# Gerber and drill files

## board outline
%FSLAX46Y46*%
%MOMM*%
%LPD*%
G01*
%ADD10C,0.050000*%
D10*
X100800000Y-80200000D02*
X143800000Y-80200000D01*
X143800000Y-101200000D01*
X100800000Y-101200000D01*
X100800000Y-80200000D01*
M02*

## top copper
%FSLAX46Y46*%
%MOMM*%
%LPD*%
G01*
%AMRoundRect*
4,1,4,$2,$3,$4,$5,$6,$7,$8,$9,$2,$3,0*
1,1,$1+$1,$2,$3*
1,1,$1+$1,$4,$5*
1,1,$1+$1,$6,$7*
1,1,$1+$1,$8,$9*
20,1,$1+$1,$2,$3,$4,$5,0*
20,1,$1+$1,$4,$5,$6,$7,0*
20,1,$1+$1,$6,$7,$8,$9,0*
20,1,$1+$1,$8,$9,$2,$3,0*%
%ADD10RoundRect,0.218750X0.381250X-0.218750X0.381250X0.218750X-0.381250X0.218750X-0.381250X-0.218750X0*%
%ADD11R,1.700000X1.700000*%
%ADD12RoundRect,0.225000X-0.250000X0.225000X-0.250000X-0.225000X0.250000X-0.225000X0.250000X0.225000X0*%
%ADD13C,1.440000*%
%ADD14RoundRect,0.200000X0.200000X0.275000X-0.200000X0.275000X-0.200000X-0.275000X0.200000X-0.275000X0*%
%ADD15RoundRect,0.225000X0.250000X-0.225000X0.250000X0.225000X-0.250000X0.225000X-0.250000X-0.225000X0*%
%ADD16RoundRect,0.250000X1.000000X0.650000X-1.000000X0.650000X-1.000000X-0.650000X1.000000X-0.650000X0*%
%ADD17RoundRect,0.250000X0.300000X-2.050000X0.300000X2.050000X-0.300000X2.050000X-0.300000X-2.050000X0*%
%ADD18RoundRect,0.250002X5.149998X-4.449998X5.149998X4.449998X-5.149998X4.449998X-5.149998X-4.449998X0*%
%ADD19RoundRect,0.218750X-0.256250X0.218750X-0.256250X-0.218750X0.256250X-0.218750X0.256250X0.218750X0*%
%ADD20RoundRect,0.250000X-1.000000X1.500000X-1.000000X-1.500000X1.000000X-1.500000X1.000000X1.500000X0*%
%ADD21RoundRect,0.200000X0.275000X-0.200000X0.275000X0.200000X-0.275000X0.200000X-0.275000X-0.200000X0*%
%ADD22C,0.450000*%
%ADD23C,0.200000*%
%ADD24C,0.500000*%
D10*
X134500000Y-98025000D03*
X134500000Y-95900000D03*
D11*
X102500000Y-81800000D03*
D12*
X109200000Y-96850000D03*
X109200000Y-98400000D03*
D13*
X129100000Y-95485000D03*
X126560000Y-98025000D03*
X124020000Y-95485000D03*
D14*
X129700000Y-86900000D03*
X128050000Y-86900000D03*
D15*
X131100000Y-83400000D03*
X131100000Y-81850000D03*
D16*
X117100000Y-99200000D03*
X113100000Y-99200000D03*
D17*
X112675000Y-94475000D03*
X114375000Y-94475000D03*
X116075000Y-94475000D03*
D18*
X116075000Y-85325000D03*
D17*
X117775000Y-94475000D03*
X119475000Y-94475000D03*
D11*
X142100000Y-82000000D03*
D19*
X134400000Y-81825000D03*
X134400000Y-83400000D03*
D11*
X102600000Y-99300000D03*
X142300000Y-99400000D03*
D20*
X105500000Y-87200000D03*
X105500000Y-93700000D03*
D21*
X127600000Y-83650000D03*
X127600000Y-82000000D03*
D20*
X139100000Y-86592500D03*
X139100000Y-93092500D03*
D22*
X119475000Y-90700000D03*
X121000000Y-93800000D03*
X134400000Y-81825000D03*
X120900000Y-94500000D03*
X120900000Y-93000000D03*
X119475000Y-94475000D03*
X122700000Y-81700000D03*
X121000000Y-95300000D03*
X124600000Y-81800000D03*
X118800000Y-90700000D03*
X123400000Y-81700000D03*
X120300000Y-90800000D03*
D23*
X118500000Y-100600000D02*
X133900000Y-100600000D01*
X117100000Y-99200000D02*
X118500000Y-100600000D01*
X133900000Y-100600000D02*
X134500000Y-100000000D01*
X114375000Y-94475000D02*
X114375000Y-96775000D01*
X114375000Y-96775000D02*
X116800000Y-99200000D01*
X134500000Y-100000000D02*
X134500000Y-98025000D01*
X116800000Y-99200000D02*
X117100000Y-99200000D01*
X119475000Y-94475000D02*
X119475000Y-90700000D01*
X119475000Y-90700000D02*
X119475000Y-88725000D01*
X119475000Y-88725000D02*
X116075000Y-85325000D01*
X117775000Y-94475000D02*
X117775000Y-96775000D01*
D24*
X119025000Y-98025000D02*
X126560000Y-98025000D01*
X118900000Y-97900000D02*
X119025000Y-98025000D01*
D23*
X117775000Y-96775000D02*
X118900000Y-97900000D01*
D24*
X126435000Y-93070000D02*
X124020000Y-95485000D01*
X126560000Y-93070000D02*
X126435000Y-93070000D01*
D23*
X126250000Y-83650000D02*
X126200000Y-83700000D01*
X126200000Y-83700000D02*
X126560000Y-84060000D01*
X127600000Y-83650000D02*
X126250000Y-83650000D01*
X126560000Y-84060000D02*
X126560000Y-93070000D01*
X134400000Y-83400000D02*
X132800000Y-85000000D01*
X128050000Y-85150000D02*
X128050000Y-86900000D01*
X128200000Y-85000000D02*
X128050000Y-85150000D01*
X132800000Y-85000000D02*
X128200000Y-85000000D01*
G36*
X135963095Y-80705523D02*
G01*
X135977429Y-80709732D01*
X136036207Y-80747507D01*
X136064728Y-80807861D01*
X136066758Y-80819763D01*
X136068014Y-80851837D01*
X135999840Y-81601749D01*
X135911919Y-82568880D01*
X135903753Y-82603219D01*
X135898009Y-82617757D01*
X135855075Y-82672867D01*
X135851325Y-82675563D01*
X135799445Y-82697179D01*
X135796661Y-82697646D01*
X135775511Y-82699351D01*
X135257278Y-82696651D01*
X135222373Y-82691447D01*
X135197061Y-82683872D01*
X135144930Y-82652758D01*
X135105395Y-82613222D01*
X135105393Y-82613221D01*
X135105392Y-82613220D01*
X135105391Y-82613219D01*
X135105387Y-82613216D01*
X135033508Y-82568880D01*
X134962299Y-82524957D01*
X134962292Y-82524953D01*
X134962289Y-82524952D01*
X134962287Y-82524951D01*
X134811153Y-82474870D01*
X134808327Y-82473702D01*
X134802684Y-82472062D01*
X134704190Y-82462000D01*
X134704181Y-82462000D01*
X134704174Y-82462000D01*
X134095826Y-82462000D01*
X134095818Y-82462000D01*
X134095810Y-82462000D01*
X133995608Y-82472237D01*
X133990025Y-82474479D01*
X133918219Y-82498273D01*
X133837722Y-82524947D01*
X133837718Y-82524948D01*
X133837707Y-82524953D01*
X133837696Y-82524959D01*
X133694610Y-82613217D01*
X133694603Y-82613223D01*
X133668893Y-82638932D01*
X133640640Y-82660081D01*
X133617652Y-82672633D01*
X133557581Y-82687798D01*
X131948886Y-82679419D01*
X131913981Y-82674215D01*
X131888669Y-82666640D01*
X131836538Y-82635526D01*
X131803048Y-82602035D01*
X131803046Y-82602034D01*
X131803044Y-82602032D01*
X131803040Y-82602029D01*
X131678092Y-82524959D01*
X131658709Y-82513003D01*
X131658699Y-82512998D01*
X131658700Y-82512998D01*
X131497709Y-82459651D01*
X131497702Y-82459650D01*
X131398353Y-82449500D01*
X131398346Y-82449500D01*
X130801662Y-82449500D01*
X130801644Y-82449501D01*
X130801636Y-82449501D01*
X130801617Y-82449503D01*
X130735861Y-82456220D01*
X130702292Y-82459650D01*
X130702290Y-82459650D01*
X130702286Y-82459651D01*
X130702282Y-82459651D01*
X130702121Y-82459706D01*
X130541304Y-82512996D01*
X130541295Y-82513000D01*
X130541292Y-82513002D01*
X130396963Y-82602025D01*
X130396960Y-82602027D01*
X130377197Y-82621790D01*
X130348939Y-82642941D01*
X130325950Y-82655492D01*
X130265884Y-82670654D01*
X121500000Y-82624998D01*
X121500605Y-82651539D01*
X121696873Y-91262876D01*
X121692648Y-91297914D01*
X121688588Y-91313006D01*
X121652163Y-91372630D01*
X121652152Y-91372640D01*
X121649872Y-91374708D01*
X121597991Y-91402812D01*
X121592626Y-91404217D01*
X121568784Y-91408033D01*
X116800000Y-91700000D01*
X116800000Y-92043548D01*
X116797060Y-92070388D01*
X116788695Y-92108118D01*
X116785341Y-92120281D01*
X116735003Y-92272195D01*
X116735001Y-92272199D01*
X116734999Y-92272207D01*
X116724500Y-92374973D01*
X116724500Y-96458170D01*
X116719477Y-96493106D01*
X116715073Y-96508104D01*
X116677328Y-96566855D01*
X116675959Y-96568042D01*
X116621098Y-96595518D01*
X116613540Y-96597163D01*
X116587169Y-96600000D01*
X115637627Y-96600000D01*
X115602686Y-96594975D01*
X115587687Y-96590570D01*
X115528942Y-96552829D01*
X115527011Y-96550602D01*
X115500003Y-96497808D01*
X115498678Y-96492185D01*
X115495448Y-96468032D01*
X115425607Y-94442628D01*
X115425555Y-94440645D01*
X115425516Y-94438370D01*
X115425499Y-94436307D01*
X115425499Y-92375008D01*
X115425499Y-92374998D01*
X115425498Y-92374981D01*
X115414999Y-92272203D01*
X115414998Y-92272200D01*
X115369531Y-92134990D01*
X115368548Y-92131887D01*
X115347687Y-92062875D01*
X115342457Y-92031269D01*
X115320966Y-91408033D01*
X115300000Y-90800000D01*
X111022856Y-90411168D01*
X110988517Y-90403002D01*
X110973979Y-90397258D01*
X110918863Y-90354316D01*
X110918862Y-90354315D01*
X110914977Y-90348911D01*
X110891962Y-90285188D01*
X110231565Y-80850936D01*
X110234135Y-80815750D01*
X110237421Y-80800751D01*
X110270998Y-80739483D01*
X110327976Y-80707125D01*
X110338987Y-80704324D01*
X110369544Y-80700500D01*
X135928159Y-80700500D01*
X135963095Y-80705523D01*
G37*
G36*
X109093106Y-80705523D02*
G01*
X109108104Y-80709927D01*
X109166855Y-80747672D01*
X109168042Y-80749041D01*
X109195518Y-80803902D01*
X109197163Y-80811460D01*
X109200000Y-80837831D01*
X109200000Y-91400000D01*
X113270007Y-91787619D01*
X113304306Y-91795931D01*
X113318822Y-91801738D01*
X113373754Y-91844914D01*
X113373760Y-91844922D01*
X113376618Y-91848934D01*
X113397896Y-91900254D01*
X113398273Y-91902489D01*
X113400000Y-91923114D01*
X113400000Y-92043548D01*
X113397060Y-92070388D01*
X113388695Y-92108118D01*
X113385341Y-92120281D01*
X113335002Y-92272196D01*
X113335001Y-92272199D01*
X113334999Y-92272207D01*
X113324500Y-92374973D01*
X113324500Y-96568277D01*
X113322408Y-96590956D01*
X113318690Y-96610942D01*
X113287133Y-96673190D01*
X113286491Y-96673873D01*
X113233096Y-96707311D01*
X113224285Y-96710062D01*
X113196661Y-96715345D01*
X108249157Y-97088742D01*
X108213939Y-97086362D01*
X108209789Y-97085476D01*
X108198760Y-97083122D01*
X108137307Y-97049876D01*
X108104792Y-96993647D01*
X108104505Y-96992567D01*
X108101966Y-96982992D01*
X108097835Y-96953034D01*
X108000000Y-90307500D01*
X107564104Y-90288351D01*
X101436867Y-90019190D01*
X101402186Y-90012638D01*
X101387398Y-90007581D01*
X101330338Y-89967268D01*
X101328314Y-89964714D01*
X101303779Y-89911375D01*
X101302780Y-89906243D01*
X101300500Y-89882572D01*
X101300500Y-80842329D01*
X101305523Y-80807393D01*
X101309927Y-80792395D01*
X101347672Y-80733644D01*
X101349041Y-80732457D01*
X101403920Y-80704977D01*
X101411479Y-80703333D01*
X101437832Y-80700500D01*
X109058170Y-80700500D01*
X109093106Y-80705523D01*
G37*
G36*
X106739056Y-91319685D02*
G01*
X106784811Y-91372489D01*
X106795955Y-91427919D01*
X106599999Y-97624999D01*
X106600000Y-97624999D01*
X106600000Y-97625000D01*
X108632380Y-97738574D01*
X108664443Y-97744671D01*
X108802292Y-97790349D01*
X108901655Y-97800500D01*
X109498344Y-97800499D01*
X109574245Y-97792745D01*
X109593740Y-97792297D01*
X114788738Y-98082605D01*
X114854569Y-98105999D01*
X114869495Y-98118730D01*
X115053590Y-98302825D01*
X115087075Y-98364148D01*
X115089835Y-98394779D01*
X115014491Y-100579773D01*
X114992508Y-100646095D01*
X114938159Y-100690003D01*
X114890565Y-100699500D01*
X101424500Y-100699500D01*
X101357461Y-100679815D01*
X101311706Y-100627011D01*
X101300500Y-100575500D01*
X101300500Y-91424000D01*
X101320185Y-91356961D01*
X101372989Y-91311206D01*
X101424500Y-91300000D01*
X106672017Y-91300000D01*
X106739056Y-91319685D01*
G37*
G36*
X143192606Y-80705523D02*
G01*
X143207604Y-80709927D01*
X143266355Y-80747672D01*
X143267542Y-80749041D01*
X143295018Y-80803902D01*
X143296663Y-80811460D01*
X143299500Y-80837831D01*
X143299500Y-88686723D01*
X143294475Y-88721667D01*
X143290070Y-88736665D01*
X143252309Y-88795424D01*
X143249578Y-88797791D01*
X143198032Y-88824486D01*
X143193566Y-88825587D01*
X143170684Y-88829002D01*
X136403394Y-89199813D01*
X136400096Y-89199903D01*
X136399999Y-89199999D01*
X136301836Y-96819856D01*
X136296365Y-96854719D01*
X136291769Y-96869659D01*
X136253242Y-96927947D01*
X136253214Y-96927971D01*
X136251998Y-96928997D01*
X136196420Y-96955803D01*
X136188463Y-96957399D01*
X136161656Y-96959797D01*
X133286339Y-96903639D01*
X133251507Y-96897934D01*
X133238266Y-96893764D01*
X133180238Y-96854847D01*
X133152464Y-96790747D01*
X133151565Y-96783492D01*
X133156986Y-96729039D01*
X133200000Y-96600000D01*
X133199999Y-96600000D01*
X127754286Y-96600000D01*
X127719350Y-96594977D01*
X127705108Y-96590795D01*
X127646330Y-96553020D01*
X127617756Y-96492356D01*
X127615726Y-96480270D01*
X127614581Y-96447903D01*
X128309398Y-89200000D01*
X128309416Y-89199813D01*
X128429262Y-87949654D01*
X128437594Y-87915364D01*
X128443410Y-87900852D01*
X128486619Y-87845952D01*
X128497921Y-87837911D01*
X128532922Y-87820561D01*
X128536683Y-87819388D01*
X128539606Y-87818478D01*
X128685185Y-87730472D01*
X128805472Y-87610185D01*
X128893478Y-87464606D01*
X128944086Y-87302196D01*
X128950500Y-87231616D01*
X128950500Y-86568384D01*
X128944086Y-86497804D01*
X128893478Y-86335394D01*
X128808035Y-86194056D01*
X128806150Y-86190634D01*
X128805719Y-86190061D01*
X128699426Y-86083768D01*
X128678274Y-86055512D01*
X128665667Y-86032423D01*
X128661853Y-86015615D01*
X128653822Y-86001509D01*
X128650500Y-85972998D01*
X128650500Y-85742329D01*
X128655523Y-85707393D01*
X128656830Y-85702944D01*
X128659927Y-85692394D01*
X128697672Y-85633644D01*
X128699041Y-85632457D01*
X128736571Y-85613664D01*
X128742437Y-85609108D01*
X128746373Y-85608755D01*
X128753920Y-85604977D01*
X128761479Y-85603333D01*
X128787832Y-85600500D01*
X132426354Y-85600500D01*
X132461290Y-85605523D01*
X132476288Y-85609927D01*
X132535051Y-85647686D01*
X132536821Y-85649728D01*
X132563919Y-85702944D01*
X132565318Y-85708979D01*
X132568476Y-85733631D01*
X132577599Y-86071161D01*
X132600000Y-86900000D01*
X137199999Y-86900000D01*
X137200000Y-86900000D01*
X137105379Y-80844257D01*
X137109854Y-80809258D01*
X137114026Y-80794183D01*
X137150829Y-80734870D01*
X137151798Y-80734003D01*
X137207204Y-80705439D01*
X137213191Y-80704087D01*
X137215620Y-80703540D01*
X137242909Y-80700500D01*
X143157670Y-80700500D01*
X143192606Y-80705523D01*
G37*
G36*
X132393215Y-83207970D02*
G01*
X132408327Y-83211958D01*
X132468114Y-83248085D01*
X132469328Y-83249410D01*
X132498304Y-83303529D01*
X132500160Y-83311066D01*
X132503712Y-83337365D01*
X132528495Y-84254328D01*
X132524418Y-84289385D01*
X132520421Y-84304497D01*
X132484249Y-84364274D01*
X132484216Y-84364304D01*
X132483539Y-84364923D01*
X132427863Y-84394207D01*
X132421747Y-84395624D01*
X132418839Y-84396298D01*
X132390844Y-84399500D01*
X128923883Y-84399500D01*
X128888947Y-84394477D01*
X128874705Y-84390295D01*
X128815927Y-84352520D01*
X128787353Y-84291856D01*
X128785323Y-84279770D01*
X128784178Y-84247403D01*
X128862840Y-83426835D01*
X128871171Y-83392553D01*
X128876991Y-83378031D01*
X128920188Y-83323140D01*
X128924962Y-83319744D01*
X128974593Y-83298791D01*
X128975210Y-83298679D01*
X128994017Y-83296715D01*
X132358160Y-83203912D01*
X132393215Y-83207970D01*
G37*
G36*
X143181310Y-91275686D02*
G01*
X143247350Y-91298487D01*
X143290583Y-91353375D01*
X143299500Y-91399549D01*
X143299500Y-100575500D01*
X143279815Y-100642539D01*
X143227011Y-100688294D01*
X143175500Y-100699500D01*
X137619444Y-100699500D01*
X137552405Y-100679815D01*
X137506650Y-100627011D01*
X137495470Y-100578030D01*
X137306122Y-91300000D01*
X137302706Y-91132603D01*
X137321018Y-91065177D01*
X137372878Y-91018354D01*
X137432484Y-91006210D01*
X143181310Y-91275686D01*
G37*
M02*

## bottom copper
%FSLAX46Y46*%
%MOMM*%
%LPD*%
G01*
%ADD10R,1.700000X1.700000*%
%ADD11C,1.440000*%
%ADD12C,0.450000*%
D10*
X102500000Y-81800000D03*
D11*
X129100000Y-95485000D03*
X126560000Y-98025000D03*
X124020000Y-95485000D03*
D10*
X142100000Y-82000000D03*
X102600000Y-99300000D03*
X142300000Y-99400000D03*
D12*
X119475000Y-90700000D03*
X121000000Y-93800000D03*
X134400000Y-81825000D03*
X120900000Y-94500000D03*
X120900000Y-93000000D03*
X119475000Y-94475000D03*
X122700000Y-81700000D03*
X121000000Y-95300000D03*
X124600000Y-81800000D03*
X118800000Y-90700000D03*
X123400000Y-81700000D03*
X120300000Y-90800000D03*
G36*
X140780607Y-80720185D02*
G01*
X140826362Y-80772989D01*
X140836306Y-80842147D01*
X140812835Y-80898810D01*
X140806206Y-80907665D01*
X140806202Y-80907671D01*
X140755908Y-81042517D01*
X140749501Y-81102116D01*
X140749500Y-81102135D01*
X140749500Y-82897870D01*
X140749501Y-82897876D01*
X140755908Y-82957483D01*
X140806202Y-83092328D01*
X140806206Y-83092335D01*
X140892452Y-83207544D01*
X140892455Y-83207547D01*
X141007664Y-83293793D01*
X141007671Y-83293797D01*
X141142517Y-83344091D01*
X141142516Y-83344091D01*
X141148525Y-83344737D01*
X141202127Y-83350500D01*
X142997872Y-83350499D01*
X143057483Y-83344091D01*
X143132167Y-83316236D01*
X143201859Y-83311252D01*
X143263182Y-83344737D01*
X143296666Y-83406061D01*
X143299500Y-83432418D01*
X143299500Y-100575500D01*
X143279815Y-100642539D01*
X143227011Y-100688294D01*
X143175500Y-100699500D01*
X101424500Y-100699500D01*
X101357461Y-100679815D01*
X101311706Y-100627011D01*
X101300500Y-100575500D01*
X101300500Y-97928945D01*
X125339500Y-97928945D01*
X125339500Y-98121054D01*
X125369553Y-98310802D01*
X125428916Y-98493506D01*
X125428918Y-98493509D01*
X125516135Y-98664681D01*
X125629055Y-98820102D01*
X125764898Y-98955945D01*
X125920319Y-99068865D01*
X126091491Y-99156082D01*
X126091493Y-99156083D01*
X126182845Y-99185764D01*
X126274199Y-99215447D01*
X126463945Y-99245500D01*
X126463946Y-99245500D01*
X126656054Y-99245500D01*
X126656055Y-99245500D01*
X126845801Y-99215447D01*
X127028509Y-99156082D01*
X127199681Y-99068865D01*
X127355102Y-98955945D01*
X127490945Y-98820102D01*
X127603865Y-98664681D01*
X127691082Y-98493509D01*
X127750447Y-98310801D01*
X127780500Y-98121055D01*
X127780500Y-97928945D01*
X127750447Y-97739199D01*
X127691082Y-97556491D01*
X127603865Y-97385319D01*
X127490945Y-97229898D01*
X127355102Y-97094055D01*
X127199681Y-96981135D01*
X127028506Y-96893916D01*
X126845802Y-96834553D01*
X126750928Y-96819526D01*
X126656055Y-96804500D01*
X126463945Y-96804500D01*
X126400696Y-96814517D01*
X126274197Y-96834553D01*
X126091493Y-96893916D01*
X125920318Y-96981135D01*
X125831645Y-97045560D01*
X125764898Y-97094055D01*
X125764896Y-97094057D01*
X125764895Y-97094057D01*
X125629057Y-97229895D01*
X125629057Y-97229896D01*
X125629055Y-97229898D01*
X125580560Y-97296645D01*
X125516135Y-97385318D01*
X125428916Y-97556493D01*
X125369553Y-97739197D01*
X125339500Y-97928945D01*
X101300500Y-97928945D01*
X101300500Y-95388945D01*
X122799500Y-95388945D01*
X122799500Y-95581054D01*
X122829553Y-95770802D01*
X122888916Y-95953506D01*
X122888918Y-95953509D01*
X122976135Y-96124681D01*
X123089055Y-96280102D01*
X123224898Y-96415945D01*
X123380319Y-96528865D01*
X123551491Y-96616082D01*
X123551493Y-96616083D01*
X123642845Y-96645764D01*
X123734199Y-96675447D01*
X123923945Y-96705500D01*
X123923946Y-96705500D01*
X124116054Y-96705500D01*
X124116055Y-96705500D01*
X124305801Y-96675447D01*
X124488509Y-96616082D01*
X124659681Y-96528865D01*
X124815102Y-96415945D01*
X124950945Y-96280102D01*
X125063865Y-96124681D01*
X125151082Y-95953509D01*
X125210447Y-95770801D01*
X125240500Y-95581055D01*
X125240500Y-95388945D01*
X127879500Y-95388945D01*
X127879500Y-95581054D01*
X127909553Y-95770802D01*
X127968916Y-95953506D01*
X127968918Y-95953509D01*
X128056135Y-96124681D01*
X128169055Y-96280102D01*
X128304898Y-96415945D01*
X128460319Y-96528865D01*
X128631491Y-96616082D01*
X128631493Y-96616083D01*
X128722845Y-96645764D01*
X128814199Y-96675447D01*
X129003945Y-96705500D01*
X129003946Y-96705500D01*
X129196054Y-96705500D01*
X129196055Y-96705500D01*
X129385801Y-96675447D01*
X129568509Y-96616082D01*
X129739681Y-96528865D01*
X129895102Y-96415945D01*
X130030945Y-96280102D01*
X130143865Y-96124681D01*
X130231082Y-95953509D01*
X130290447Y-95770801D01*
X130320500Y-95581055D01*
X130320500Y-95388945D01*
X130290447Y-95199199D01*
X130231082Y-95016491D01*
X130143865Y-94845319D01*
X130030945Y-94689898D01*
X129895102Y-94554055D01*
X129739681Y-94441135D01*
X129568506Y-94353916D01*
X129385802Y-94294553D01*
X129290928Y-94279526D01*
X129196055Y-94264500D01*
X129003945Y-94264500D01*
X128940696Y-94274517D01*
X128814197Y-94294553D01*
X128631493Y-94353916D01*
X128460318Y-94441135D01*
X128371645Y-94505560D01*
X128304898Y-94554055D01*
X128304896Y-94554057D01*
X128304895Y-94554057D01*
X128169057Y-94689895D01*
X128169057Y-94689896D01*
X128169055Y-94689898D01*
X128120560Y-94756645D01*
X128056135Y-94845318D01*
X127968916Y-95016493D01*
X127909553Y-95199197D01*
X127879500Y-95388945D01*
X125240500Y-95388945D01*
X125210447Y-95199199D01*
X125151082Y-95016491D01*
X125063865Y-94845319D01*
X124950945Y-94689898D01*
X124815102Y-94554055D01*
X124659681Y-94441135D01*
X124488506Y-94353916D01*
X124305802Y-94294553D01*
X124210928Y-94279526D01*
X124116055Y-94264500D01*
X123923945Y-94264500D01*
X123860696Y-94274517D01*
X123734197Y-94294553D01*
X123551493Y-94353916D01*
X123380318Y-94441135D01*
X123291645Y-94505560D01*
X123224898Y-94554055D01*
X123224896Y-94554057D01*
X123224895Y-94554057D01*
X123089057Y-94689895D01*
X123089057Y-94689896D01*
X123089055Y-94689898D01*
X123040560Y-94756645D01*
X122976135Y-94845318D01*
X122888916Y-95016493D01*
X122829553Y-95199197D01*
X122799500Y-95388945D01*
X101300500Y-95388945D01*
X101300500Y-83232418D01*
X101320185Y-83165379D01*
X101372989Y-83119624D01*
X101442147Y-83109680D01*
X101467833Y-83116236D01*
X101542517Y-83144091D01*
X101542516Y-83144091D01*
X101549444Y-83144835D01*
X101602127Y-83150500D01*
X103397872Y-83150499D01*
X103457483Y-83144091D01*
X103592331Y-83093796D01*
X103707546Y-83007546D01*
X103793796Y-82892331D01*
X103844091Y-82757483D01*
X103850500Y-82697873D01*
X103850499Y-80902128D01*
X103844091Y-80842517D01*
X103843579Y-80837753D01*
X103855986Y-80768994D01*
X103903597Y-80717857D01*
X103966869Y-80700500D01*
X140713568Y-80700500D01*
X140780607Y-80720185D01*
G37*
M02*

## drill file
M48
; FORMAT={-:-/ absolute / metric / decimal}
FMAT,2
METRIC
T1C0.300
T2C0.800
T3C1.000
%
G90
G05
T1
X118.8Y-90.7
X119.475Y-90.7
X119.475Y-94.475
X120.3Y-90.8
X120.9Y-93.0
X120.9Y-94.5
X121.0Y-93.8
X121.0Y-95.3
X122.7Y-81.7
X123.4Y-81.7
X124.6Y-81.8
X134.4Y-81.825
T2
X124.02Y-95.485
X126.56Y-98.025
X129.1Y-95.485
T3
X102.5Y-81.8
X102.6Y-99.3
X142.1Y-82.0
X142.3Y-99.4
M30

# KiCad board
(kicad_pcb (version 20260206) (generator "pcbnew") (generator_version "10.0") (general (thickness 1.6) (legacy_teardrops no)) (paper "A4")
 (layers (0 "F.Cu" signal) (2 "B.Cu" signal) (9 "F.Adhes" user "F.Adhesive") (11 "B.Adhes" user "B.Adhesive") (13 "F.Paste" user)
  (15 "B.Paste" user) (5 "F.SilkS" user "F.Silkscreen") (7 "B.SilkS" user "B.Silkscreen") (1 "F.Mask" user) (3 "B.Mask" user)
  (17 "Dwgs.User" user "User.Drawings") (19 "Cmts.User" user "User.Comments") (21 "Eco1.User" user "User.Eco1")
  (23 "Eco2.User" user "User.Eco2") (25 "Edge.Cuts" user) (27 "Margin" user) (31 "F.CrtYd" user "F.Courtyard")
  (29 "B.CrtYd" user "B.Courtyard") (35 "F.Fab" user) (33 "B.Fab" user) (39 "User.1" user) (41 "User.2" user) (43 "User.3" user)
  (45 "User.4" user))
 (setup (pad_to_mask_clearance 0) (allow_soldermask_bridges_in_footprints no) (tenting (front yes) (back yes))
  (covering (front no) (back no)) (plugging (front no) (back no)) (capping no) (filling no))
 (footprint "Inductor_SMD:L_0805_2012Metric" (layer "F.Cu") (at 134.5 96.9625 90)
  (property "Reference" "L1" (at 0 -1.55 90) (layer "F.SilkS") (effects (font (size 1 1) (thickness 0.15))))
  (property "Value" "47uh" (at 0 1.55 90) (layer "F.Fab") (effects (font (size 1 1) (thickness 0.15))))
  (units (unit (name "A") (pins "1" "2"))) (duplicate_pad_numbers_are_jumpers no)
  (pad "1" smd roundrect (at -1.0625 0 90) (size 0.875 1.2) (layers "F.Cu" "F.Mask" "F.Paste") (roundrect_rratio 0.25) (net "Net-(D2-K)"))
  (pad "2" smd roundrect (at 1.0625 0 90) (size 0.875 1.2) (layers "F.Cu" "F.Mask" "F.Paste") (roundrect_rratio 0.25) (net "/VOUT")))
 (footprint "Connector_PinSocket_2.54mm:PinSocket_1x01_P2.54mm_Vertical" (layer "F.Cu") (at 102.5 81.8)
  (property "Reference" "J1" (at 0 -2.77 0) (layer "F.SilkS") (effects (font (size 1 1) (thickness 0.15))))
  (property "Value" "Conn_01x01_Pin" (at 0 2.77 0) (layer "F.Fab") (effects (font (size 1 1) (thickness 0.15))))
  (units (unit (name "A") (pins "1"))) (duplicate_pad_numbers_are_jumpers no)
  (pad "1" thru_hole rect (at 0 0) (size 1.7 1.7) (drill 1) (layers "*.Cu" "*.Mask") (remove_unused_layers no) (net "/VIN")))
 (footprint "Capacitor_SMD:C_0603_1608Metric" (layer "F.Cu") (at 109.2 97.625 -90)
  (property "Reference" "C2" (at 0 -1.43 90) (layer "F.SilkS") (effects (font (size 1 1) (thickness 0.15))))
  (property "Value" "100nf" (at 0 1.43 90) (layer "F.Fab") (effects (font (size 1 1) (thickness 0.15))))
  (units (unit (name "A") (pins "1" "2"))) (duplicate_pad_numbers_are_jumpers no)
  (pad "1" smd roundrect (at -0.775 0 270) (size 0.9 0.95) (layers "F.Cu" "F.Mask" "F.Paste") (roundrect_rratio 0.25) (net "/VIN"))
  (pad "2" smd roundrect (at 0.775 0 270) (size 0.9 0.95) (layers "F.Cu" "F.Mask" "F.Paste") (roundrect_rratio 0.25) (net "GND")))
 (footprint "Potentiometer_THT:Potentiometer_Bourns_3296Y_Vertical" (layer "F.Cu") (at 129.1 95.485)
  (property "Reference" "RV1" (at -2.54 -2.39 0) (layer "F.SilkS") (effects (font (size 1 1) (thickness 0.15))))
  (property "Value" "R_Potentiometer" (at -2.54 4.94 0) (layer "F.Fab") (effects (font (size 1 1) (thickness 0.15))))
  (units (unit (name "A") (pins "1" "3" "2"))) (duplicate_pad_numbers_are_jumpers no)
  (pad "1" thru_hole circle (at 0 0) (size 1.44 1.44) (drill 0.8) (layers "*.Cu" "*.Mask") (remove_unused_layers no) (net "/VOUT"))
  (pad "2" thru_hole circle (at -2.54 2.54) (size 1.44 1.44) (drill 0.8) (layers "*.Cu" "*.Mask") (remove_unused_layers no)
   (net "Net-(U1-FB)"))
  (pad "3" thru_hole circle (at -5.08 0) (size 1.44 1.44) (drill 0.8) (layers "*.Cu" "*.Mask") (remove_unused_layers no)
   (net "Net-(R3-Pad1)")))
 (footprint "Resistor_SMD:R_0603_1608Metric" (layer "F.Cu") (at 128.875 86.9 180)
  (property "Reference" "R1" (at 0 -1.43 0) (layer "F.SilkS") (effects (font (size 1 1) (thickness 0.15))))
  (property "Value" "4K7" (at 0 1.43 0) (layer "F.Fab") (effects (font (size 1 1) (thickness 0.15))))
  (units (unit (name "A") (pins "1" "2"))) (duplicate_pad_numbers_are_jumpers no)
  (pad "1" smd roundrect (at -0.825 0 180) (size 0.8 0.95) (layers "F.Cu" "F.Mask" "F.Paste") (roundrect_rratio 0.25) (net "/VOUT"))
  (pad "2" smd roundrect (at 0.825 0 180) (size 0.8 0.95) (layers "F.Cu" "F.Mask" "F.Paste") (roundrect_rratio 0.25) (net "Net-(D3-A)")))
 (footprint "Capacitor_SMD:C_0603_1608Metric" (layer "F.Cu") (at 131.1 82.625 90)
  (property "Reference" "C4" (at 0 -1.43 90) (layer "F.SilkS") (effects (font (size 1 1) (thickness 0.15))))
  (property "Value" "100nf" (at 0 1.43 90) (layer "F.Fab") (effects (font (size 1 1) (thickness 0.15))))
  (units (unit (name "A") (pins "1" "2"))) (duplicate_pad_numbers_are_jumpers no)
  (pad "1" smd roundrect (at -0.775 0 90) (size 0.9 0.95) (layers "F.Cu" "F.Mask" "F.Paste") (roundrect_rratio 0.25) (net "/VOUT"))
  (pad "2" smd roundrect (at 0.775 0 90) (size 0.9 0.95) (layers "F.Cu" "F.Mask" "F.Paste") (roundrect_rratio 0.25) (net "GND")))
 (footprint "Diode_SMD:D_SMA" (layer "F.Cu") (at 115.1 99.2 180)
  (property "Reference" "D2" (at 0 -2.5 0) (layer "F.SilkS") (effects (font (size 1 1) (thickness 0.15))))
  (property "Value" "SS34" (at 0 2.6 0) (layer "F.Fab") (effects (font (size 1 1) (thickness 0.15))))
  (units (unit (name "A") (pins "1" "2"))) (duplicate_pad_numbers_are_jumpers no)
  (pad "1" smd roundrect (at -2 0 180) (size 2.5 1.8) (layers "F.Cu" "F.Mask" "F.Paste") (roundrect_rratio 0.1388888889) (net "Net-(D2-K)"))
  (pad "2" smd roundrect (at 2 0 180) (size 2.5 1.8) (layers "F.Cu" "F.Mask" "F.Paste") (roundrect_rratio 0.1388888889) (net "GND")))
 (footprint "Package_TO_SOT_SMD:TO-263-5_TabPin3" (layer "F.Cu") (at 116.075 86.825 90)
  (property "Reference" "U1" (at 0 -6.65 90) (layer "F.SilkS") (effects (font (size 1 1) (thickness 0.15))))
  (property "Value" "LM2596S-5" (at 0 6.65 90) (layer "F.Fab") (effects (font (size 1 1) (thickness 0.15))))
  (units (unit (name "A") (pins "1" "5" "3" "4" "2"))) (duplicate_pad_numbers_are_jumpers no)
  (pad "" smd roundrect (at -0.925 -2.775 90) (size 4.55 5.25) (layers "F.Paste") (roundrect_rratio 0.054945))
  (pad "" smd roundrect (at -0.925 2.775 90) (size 4.55 5.25) (layers "F.Paste") (roundrect_rratio 0.054945))
  (pad "" smd roundrect (at 3.925 -2.775 90) (size 4.55 5.25) (layers "F.Paste") (roundrect_rratio 0.054945))
  (pad "" smd roundrect (at 3.925 2.775 90) (size 4.55 5.25) (layers "F.Paste") (roundrect_rratio 0.054945))
  (pad "1" smd roundrect (at -7.65 -3.4 90) (size 4.6 1.1) (layers "F.Cu" "F.Mask" "F.Paste") (roundrect_rratio 0.227273) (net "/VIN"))
  (pad "2" smd roundrect (at -7.65 -1.7 90) (size 4.6 1.1) (layers "F.Cu" "F.Mask" "F.Paste") (roundrect_rratio 0.227273) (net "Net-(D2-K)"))
  (pad "3" smd roundrect (at -7.65 0 90) (size 4.6 1.1) (layers "F.Cu" "F.Mask" "F.Paste") (roundrect_rratio 0.227273) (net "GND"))
  (pad "3" smd roundrect (at 1.5 0 90) (size 9.4 10.8) (layers "F.Cu" "F.Mask") (roundrect_rratio 0.026596) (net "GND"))
  (pad "4" smd roundrect (at -7.65 1.7 90) (size 4.6 1.1) (layers "F.Cu" "F.Mask" "F.Paste") (roundrect_rratio 0.227273) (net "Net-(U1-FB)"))
  (pad "5" smd roundrect (at -7.65 3.4 90) (size 4.6 1.1) (layers "F.Cu" "F.Mask" "F.Paste") (roundrect_rratio 0.227273) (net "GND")))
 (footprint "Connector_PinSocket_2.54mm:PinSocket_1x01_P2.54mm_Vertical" (layer "F.Cu") (at 142.1 82)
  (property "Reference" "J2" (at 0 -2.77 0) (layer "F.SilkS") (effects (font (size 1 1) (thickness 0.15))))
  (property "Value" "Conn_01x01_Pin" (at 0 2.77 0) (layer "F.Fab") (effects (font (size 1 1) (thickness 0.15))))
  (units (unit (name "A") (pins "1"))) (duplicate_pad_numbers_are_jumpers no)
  (pad "1" thru_hole rect (at 0 0) (size 1.7 1.7) (drill 1) (layers "*.Cu" "*.Mask") (remove_unused_layers no) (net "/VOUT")))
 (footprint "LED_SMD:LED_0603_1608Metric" (layer "F.Cu") (at 134.4 82.6125 -90)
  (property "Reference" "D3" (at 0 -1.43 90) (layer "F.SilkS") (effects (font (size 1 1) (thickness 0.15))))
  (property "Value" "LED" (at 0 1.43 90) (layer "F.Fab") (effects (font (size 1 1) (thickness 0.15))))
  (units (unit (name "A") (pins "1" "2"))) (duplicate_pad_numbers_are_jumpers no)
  (pad "1" smd roundrect (at -0.7875 0 270) (size 0.875 0.95) (layers "F.Cu" "F.Mask" "F.Paste") (roundrect_rratio 0.25) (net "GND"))
  (pad "2" smd roundrect (at 0.7875 0 270) (size 0.875 0.95) (layers "F.Cu" "F.Mask" "F.Paste") (roundrect_rratio 0.25) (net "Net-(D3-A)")))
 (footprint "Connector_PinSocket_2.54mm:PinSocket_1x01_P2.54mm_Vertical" (layer "F.Cu") (at 102.6 99.3)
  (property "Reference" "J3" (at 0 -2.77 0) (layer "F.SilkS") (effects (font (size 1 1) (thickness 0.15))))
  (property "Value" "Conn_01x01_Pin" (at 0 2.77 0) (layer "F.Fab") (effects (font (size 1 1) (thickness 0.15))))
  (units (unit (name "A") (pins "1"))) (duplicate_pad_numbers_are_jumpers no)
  (pad "1" thru_hole rect (at 0 0) (size 1.7 1.7) (drill 1) (layers "*.Cu" "*.Mask") (remove_unused_layers no) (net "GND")))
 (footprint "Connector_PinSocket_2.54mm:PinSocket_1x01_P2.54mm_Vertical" (layer "F.Cu") (at 142.3 99.4)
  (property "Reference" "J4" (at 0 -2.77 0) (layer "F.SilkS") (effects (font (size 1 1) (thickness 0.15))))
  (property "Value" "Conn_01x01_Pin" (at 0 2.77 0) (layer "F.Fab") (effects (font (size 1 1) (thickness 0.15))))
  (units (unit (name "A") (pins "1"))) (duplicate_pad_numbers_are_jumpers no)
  (pad "1" thru_hole rect (at 0 0) (size 1.7 1.7) (drill 1) (layers "*.Cu" "*.Mask") (remove_unused_layers no) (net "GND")))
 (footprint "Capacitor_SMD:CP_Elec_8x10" (layer "F.Cu") (at 105.5 90.45 -90)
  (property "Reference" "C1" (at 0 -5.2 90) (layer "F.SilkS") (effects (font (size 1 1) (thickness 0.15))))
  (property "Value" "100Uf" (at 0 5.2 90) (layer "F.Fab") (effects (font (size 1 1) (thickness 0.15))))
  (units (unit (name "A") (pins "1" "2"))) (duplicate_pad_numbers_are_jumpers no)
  (pad "1" smd roundrect (at -3.25 0 270) (size 3.5 2.5) (layers "F.Cu" "F.Mask" "F.Paste") (roundrect_rratio 0.1) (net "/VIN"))
  (pad "2" smd roundrect (at 3.25 0 270) (size 3.5 2.5) (layers "F.Cu" "F.Mask" "F.Paste") (roundrect_rratio 0.1) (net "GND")))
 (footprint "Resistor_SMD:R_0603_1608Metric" (layer "F.Cu") (at 127.6 82.825 90)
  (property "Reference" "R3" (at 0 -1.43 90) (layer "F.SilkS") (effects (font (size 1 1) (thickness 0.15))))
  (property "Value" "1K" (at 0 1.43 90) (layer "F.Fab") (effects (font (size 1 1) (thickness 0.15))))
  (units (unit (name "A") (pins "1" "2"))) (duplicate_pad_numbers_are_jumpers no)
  (pad "1" smd roundrect (at -0.825 0 90) (size 0.8 0.95) (layers "F.Cu" "F.Mask" "F.Paste") (roundrect_rratio 0.25) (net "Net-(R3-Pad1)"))
  (pad "2" smd roundrect (at 0.825 0 90) (size 0.8 0.95) (layers "F.Cu" "F.Mask" "F.Paste") (roundrect_rratio 0.25) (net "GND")))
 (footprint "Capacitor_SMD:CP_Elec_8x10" (layer "F.Cu") (at 139.1 89.8425 -90)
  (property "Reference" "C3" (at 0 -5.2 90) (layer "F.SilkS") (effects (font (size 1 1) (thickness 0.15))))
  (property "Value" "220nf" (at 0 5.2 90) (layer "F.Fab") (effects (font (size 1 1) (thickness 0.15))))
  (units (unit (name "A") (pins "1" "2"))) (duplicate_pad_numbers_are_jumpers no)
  (pad "1" smd roundrect (at -3.25 0 270) (size 3.5 2.5) (layers "F.Cu" "F.Mask" "F.Paste") (roundrect_rratio 0.1) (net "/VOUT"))
  (pad "2" smd roundrect (at 3.25 0 270) (size 3.5 2.5) (layers "F.Cu" "F.Mask" "F.Paste") (roundrect_rratio 0.1) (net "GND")))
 (gr_rect (start 100.8 80.2) (end 143.8 101.2) (stroke (width 0.05) (type solid)) (fill no) (layer "Edge.Cuts"))
 (segment (start 118.5 100.6) (end 133.9 100.6) (width 0.2) (layer "F.Cu") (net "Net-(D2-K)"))
 (segment (start 117.1 99.2) (end 118.5 100.6) (width 0.2) (layer "F.Cu") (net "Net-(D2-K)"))
 (segment (start 133.9 100.6) (end 134.5 100) (width 0.2) (layer "F.Cu") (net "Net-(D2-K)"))
 (segment (start 114.375 94.475) (end 114.375 96.775) (width 0.2) (layer "F.Cu") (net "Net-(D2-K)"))
 (segment (start 114.375 96.775) (end 116.8 99.2) (width 0.2) (layer "F.Cu") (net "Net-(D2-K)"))
 (segment (start 134.5 100) (end 134.5 98.025) (width 0.2) (layer "F.Cu") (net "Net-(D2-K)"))
 (segment (start 116.8 99.2) (end 117.1 99.2) (width 0.2) (layer "F.Cu") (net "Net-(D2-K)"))
 (segment (start 119.475 94.475) (end 119.475 90.7) (width 0.2) (layer "F.Cu") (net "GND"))
 (segment (start 119.475 90.7) (end 119.475 88.725) (width 0.2) (layer "F.Cu") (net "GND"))
 (segment (start 119.475 88.725) (end 116.075 85.325) (width 0.2) (layer "F.Cu") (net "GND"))
 (via (at 119.475 90.7) (size 0.45) (drill 0.3) (layers "F.Cu" "B.Cu") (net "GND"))
 (via (at 121 93.8) (size 0.45) (drill 0.3) (layers "F.Cu" "B.Cu") (free yes) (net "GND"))
 (via (at 134.4 81.825) (size 0.45) (drill 0.3) (layers "F.Cu" "B.Cu") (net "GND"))
 (via (at 120.9 94.5) (size 0.45) (drill 0.3) (layers "F.Cu" "B.Cu") (free yes) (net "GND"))
 (via (at 120.9 93) (size 0.45) (drill 0.3) (layers "F.Cu" "B.Cu") (free yes) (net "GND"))
 (via (at 119.475 94.475) (size 0.45) (drill 0.3) (layers "F.Cu" "B.Cu") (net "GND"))
 (via (at 122.7 81.7) (size 0.45) (drill 0.3) (layers "F.Cu" "B.Cu") (free yes) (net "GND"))
 (via (at 121 95.3) (size 0.45) (drill 0.3) (layers "F.Cu" "B.Cu") (free yes) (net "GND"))
 (via (at 124.6 81.8) (size 0.45) (drill 0.3) (layers "F.Cu" "B.Cu") (free yes) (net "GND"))
 (via (at 118.8 90.7) (size 0.45) (drill 0.3) (layers "F.Cu" "B.Cu") (free yes) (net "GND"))
 (via (at 123.4 81.7) (size 0.45) (drill 0.3) (layers "F.Cu" "B.Cu") (free yes) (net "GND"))
 (via (at 120.3 90.8) (size 0.45) (drill 0.3) (layers "F.Cu" "B.Cu") (free yes) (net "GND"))
 (segment (start 117.775 94.475) (end 117.775 96.775) (width 0.2) (layer "F.Cu") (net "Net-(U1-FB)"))
 (segment (start 119.025 98.025) (end 126.56 98.025) (width 0.5) (layer "F.Cu") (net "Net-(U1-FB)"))
 (segment (start 118.9 97.9) (end 119.025 98.025) (width 0.5) (layer "F.Cu") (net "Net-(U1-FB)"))
 (segment (start 117.775 96.775) (end 118.9 97.9) (width 0.2) (layer "F.Cu") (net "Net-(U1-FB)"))
 (segment (start 126.435 93.07) (end 124.02 95.485) (width 0.5) (layer "F.Cu") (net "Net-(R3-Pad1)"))
 (segment (start 126.56 93.07) (end 126.435 93.07) (width 0.5) (layer "F.Cu") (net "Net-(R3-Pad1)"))
 (segment (start 126.25 83.65) (end 126.2 83.7) (width 0.2) (layer "F.Cu") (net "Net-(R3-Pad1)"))
 (segment (start 126.2 83.7) (end 126.56 84.06) (width 0.2) (layer "F.Cu") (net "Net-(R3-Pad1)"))
 (segment (start 127.6 83.65) (end 126.25 83.65) (width 0.2) (layer "F.Cu") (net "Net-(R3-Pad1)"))
 (segment (start 126.56 84.06) (end 126.56 93.07) (width 0.2) (layer "F.Cu") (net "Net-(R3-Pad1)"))
 (segment (start 134.4 83.4) (end 132.8 85) (width 0.2) (layer "F.Cu") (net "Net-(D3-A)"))
 (segment (start 128.05 85.15) (end 128.05 86.9) (width 0.2) (layer "F.Cu") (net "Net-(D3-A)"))
 (segment (start 128.2 85) (end 128.05 85.15) (width 0.2) (layer "F.Cu") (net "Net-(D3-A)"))
 (segment (start 132.8 85) (end 128.2 85) (width 0.2) (layer "F.Cu") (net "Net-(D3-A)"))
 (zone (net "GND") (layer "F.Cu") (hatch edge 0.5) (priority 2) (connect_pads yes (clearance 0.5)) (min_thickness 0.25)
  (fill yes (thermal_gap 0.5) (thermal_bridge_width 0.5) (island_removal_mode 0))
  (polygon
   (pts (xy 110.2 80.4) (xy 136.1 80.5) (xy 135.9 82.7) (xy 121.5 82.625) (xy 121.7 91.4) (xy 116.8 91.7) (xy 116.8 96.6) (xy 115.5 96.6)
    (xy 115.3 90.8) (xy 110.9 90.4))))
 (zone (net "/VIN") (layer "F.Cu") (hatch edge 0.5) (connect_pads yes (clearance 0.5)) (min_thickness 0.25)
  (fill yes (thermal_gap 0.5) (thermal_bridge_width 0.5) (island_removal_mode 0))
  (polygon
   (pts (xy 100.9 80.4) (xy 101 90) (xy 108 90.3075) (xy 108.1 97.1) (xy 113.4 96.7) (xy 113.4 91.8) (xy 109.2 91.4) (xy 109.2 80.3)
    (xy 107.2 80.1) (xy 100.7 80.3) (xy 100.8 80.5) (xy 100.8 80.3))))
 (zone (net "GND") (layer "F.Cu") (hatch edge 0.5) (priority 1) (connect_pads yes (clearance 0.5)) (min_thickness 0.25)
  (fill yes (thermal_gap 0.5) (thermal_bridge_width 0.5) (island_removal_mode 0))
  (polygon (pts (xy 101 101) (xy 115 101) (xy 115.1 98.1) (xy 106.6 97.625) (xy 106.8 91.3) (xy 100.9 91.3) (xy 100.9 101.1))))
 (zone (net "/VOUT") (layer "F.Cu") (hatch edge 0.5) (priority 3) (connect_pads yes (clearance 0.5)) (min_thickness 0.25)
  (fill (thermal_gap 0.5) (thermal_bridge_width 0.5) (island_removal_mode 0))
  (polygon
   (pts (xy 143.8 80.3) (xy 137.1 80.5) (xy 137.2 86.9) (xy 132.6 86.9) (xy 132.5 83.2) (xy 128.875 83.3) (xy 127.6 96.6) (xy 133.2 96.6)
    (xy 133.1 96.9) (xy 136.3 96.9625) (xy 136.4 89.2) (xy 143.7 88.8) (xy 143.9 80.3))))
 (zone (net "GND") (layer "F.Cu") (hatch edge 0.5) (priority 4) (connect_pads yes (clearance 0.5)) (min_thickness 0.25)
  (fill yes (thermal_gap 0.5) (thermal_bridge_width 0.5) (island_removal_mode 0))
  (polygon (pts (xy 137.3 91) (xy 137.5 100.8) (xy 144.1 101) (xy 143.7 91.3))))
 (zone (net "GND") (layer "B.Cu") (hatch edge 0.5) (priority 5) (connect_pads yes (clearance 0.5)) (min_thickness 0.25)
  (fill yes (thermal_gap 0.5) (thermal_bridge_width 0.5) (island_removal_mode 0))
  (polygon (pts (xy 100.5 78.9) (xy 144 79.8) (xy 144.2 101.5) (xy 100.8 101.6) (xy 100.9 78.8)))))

